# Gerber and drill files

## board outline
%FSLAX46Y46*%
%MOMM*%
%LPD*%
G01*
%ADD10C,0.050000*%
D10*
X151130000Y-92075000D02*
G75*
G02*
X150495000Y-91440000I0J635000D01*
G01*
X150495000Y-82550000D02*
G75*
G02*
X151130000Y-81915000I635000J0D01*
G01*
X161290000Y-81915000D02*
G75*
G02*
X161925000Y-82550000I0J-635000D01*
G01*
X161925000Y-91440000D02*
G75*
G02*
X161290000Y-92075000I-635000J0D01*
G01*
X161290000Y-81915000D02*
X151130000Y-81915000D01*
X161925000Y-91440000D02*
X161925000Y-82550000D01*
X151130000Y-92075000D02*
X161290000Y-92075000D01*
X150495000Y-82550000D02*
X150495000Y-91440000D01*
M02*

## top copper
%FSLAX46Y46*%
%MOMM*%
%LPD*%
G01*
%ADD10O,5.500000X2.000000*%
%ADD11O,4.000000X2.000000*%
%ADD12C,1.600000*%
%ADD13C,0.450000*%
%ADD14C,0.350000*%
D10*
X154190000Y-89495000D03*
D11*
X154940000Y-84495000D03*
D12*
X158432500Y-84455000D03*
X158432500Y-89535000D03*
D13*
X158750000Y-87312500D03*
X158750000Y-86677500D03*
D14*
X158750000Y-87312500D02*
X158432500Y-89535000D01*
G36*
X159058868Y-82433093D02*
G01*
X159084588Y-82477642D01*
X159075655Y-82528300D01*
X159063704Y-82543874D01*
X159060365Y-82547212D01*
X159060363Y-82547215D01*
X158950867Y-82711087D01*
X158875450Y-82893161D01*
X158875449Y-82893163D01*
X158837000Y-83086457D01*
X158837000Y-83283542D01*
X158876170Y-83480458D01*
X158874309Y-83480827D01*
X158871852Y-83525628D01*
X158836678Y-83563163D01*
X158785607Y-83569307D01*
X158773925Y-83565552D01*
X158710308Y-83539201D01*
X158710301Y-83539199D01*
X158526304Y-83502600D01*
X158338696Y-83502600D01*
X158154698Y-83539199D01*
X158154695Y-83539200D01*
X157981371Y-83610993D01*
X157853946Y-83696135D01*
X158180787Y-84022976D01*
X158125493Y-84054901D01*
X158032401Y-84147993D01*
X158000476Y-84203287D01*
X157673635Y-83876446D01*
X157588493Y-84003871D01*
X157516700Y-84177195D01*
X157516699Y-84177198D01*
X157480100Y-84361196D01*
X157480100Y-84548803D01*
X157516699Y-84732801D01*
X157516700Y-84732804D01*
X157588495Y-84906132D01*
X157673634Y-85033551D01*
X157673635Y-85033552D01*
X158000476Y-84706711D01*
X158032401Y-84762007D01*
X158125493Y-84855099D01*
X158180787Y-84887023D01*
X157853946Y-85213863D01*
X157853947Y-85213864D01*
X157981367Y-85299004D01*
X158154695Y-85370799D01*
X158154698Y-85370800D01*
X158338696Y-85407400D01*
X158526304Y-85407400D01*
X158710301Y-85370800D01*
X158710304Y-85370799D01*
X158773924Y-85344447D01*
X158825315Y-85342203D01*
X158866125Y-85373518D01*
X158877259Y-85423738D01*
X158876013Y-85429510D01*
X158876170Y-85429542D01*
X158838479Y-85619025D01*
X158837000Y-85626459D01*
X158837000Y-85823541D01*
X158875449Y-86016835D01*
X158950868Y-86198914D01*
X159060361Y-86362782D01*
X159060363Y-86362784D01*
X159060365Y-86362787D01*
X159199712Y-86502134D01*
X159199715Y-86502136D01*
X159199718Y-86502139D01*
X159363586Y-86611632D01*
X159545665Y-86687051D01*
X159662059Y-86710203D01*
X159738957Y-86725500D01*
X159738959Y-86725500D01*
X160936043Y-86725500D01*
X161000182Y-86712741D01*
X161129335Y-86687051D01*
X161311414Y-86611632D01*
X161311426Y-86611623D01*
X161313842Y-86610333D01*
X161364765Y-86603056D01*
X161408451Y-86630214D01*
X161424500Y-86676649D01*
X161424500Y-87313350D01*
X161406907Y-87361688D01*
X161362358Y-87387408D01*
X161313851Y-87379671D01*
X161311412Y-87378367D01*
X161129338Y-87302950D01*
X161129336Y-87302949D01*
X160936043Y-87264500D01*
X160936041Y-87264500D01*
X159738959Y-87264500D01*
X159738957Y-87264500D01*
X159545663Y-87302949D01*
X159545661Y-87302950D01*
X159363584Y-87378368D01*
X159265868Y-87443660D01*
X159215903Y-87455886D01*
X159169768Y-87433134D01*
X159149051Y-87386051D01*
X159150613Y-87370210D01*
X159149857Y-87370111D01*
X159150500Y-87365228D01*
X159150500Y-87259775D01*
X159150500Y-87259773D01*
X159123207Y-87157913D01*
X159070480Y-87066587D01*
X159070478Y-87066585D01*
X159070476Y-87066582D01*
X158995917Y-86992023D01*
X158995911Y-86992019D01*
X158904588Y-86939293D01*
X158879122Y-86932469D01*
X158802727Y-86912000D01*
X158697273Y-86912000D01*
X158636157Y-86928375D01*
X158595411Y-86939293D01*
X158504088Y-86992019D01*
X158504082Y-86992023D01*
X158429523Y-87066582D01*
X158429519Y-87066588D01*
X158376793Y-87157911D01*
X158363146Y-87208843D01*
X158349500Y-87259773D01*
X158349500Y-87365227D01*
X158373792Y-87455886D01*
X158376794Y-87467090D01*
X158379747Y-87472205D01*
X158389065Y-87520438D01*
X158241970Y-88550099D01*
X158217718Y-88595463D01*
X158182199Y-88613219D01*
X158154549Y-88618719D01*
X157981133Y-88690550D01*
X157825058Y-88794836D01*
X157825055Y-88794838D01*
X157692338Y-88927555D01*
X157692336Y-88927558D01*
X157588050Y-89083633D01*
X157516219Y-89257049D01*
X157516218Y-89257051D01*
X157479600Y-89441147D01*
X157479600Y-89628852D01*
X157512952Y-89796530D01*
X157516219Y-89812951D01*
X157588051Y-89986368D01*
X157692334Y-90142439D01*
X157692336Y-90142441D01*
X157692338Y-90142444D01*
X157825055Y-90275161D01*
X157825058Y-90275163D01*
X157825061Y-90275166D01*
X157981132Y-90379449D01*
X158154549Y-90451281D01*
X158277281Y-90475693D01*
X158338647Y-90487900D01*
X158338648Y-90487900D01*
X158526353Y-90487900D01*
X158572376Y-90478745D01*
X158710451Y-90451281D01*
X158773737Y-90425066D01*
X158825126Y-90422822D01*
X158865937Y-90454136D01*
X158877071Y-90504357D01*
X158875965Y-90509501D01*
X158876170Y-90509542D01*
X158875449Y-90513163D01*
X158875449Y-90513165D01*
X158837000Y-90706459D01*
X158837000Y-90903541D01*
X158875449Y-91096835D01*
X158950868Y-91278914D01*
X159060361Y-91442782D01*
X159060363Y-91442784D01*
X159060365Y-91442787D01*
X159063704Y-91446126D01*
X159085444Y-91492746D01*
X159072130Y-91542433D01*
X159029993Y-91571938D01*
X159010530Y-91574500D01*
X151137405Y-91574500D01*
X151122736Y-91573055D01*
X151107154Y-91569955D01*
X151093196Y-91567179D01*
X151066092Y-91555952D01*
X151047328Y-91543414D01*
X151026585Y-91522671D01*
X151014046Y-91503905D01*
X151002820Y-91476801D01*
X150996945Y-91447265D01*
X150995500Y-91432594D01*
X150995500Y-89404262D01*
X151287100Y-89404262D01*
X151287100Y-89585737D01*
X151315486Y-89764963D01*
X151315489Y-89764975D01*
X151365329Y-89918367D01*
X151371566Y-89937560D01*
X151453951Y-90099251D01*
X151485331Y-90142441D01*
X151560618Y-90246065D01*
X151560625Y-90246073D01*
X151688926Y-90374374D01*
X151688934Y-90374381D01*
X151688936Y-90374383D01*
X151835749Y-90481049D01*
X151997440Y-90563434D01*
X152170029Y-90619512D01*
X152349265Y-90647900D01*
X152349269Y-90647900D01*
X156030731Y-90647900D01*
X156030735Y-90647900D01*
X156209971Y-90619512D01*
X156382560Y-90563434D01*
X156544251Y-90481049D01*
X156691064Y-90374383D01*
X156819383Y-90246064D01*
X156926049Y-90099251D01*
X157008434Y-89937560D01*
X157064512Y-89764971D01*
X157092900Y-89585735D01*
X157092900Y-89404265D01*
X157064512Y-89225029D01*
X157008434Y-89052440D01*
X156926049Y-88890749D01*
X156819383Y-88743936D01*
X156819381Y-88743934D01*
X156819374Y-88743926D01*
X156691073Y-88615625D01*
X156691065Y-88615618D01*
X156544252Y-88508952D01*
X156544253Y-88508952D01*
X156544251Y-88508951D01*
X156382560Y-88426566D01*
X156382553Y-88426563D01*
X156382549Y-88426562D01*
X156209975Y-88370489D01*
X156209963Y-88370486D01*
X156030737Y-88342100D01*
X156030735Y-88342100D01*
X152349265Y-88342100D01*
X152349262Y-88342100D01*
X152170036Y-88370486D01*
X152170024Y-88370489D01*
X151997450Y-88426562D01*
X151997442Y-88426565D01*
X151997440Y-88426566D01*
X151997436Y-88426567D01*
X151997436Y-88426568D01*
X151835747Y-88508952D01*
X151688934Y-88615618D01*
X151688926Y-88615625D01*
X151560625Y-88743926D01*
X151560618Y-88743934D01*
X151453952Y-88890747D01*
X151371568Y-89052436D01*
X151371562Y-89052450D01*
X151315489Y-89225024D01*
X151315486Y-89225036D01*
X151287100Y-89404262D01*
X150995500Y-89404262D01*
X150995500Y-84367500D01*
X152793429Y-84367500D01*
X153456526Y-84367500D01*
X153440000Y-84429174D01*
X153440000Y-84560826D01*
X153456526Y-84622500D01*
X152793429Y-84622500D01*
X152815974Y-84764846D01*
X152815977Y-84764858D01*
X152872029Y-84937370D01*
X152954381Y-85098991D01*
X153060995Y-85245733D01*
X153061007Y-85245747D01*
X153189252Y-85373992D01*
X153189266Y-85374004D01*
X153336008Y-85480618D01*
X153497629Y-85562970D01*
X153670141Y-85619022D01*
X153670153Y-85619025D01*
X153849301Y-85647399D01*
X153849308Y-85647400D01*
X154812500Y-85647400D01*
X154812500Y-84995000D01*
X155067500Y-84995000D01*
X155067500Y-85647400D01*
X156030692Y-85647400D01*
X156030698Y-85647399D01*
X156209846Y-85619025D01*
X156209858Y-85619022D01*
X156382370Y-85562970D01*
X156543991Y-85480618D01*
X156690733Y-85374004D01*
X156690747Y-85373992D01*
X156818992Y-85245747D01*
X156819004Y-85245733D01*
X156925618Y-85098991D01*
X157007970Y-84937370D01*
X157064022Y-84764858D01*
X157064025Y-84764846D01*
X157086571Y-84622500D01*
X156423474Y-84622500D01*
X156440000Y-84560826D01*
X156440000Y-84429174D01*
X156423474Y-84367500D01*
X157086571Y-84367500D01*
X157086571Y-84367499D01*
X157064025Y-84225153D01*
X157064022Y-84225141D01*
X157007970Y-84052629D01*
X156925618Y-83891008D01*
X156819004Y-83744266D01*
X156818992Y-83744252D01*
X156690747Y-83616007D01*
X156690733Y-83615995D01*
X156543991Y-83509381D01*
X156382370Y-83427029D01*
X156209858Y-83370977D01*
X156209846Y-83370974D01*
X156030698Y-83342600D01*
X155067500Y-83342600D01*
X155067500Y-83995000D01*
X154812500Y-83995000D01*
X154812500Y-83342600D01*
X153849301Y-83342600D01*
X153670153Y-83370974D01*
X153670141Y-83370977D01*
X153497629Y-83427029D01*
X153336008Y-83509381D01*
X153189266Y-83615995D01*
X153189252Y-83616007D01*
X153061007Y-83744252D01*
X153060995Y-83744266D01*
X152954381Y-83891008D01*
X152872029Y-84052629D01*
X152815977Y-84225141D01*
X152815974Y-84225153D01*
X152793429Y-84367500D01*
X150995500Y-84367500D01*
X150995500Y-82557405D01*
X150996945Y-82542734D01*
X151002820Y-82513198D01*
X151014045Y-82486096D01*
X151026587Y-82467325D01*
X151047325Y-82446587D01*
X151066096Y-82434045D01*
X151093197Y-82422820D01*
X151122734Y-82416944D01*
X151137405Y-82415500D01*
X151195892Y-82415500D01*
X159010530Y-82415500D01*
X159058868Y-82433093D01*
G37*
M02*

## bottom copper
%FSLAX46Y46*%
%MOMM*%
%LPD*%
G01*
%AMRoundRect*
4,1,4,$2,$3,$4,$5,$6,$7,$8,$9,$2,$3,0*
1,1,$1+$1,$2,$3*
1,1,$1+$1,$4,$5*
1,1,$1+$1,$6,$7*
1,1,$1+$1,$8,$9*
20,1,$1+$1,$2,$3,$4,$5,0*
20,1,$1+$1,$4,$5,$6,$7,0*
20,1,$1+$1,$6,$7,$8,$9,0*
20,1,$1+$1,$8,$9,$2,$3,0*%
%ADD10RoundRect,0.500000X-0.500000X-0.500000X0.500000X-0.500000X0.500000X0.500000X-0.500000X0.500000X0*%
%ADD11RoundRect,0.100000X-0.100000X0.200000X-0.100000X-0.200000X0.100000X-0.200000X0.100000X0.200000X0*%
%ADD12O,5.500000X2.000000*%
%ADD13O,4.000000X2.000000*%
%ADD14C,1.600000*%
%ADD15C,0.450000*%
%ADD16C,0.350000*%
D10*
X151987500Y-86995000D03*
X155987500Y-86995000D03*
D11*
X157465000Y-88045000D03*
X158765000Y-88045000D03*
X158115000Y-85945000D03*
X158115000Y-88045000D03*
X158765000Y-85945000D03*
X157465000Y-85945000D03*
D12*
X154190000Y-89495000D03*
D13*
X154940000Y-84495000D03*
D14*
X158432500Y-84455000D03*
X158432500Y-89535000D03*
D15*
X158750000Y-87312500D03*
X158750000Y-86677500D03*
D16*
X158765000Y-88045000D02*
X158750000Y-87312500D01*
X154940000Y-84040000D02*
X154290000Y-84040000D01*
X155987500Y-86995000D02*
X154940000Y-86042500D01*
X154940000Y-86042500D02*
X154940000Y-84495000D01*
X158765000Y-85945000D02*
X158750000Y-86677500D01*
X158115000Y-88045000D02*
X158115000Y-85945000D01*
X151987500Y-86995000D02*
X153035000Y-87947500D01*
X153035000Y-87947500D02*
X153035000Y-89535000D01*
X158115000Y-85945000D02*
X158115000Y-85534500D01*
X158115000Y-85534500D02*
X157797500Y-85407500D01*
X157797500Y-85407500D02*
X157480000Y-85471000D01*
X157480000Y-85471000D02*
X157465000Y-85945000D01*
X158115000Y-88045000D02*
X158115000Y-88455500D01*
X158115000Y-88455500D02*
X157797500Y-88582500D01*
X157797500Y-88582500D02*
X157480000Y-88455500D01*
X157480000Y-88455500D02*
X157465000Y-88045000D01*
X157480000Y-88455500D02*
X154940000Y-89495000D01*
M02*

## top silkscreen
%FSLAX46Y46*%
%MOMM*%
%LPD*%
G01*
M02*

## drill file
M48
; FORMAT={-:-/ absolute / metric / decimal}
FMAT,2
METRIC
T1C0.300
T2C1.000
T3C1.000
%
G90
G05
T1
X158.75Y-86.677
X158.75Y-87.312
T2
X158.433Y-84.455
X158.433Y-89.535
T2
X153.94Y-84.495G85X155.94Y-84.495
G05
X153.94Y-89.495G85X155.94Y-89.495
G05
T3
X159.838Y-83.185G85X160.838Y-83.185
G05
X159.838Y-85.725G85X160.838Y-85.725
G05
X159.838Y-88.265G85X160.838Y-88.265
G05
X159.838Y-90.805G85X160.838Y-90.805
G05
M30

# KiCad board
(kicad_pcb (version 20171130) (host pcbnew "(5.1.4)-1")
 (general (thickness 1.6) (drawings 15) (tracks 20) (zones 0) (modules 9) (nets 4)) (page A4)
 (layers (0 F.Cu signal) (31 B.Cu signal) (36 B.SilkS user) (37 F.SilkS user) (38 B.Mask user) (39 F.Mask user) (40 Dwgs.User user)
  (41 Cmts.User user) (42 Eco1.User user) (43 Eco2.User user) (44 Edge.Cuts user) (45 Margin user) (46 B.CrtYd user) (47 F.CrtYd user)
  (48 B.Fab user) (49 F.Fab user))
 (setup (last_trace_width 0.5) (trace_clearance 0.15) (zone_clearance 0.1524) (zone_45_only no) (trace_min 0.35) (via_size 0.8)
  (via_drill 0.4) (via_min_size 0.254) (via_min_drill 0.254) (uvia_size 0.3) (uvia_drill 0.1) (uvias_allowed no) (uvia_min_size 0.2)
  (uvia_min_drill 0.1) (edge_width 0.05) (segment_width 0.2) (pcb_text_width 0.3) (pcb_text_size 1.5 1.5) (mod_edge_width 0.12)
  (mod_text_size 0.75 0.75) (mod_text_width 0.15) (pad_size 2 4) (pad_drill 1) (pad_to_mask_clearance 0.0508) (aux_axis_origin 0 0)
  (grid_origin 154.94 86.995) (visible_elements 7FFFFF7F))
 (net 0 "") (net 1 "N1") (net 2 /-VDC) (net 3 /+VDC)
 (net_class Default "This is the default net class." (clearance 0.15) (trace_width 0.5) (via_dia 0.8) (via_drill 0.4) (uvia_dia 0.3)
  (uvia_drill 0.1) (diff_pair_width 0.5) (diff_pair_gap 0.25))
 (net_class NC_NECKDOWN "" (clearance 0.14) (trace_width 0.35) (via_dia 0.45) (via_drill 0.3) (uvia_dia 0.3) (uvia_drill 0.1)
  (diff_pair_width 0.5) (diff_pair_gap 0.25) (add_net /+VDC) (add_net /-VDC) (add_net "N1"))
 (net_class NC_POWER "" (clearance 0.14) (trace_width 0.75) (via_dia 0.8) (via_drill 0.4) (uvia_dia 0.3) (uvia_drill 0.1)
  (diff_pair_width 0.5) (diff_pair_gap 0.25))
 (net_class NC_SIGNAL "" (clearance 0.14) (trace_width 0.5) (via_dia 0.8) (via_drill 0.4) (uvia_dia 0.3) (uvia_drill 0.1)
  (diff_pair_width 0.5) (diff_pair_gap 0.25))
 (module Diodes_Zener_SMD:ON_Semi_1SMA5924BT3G (layer B.Cu) (at 153.9875 86.995)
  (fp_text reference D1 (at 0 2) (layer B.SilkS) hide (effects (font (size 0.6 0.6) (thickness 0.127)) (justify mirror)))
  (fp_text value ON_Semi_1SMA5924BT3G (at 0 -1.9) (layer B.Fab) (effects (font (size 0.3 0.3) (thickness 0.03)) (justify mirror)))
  (pad 2 smd roundrect (at -2 0) (size 2 2) (layers B.Cu B.Paste B.Mask) (roundrect_rratio 0.25) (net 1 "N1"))
  (pad 1 smd roundrect (at 2 0) (size 2 2) (layers B.Cu B.Paste B.Mask) (roundrect_rratio 0.25) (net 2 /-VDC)))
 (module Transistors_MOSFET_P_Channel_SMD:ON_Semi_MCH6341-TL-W (layer B.Cu) (at 158.115 86.995 270)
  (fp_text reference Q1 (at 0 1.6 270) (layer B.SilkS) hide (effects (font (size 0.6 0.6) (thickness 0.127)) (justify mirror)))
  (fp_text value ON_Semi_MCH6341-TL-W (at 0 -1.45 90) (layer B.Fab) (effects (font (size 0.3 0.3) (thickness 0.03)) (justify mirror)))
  (pad 6 smd roundrect (at 1.05 0.65 270) (size 0.6 0.4) (layers B.Cu B.Paste B.Mask) (roundrect_rratio 0.25) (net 1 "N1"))
  (pad 4 smd roundrect (at 1.05 -0.65 270) (size 0.6 0.4) (layers B.Cu B.Paste B.Mask) (roundrect_rratio 0.25) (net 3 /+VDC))
  (pad 2 smd roundrect (at -1.05 0 270) (size 0.6 0.4) (layers B.Cu B.Paste B.Mask) (roundrect_rratio 0.25) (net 1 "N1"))
  (pad 5 smd roundrect (at 1.05 0 270) (size 0.6 0.4) (layers B.Cu B.Paste B.Mask) (roundrect_rratio 0.25) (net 1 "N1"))
  (pad 3 smd roundrect (at -1.05 -0.65 270) (size 0.6 0.4) (layers B.Cu B.Paste B.Mask) (roundrect_rratio 0.25) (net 2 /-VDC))
  (pad 1 smd roundrect (at -1.05 0.65 270) (size 0.6 0.4) (layers B.Cu B.Paste B.Mask) (roundrect_rratio 0.25) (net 1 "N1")))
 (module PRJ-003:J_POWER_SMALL (layer F.Cu) (at 154.94 86.995)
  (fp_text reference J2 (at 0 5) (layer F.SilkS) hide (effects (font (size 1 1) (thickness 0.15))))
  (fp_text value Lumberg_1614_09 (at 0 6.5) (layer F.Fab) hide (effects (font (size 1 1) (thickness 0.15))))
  (pad 2 thru_hole oval (at 0 2.5) (size 5.5 2) (drill oval 3 1 (offset -0.75 0)) (layers *.Cu *.Mask) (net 1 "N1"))
  (pad 1 thru_hole oval (at 0 -2.5 90) (size 2 4) (drill oval 1 3) (layers *.Cu *.Mask) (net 2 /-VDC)))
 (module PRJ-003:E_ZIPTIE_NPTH (layer F.Cu) (at 160.3375 88.265 90)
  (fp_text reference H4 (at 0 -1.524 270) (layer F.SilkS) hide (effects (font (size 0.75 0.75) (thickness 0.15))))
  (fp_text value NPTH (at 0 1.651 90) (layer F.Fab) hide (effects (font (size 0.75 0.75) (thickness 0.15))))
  (pad "" np_thru_hole oval (at 0 0 90) (size 1 2) (drill oval 1 2) (layers *.Cu *.Mask)))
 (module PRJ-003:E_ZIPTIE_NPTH (layer F.Cu) (at 160.3375 85.725 90)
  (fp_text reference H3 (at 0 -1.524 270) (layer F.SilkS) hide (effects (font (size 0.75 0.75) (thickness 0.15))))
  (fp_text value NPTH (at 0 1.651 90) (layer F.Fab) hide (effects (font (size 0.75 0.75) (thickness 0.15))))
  (pad "" np_thru_hole oval (at 0 0 90) (size 1 2) (drill oval 1 2) (layers *.Cu *.Mask)))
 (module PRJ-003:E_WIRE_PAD (layer B.Cu) (at 158.4325 84.455)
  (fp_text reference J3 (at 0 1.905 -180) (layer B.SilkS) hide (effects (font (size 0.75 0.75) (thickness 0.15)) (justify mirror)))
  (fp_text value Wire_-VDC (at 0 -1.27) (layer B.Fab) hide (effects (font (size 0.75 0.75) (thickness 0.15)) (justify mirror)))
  (pad "" connect circle (at 0 0) (size 1 1) (layers B.Mask))
  (pad 1 thru_hole circle (at 0 0) (size 1.6 1.6) (drill 1) (layers F.Cu F.Mask) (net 2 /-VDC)))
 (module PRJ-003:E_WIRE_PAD (layer B.Cu) (at 158.4325 89.535)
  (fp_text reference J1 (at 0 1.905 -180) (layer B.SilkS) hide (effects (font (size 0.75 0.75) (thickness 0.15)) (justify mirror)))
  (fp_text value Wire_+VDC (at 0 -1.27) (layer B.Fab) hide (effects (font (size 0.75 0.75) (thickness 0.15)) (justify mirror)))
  (pad "" connect circle (at 0 0) (size 1 1) (layers B.Mask))
  (pad 1 thru_hole circle (at 0 0) (size 1.6 1.6) (drill 1) (layers F.Cu F.Mask) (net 3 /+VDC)))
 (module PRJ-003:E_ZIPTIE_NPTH (layer F.Cu) (at 160.3375 90.805 90)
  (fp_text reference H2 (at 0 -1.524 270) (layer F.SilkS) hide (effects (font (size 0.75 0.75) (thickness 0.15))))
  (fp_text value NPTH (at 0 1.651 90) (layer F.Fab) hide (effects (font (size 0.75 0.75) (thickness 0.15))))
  (pad "" np_thru_hole oval (at 0 0 90) (size 1 2) (drill oval 1 2) (layers *.Cu *.Mask)))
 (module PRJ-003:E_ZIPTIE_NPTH (layer F.Cu) (at 160.3375 83.185 90)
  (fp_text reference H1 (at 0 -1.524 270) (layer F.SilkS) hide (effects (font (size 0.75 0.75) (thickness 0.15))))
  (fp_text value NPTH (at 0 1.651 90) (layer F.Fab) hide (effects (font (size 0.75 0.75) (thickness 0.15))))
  (pad "" np_thru_hole oval (at 0 0 90) (size 1 2) (drill oval 1 2) (layers *.Cu *.Mask)))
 (gr_arc (start 151.13 91.44) (end 150.495 91.44) (angle -90) (layer Edge.Cuts) (width 0.05))
 (gr_arc (start 151.13 82.55) (end 151.13 81.915) (angle -90) (layer Edge.Cuts) (width 0.05))
 (gr_arc (start 161.29 82.55) (end 161.925 82.55) (angle -90) (layer Edge.Cuts) (width 0.05))
 (gr_arc (start 161.29 91.44) (end 161.29 92.075) (angle -90) (layer Edge.Cuts) (width 0.05))
 (gr_line (start 161.29 81.915) (end 151.13 81.915) (layer Edge.Cuts) (width 0.05))
 (gr_line (start 161.925 91.44) (end 161.925 82.55) (layer Edge.Cuts) (width 0.05))
 (gr_line (start 151.13 92.075) (end 161.29 92.075) (layer Edge.Cuts) (width 0.05))
 (gr_line (start 150.495 82.55) (end 150.495 91.44) (layer Edge.Cuts) (width 0.05))
 (via (at 158.75 87.3125) (size 0.45) (drill 0.3) (layers F.Cu B.Cu) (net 3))
 (segment (start 158.765 88.045) (end 158.75 87.3125) (width 0.35) (layer B.Cu) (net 3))
 (segment (start 158.75 87.3125) (end 158.4325 89.535) (width 0.35) (layer F.Cu) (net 3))
 (segment (start 154.94 84.04) (end 154.29 84.04) (width 0.35) (layer B.Cu) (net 2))
 (segment (start 155.9875 86.995) (end 154.94 86.0425) (width 0.35) (layer B.Cu) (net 2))
 (segment (start 154.94 86.0425) (end 154.94 84.495) (width 0.35) (layer B.Cu) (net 2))
 (segment (start 158.765 85.945) (end 158.75 86.6775) (width 0.35) (layer B.Cu) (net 2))
 (via (at 158.75 86.6775) (size 0.45) (drill 0.3) (layers F.Cu B.Cu) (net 2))
 (segment (start 158.115 88.045) (end 158.115 85.945) (width 0.35) (layer B.Cu) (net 1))
 (segment (start 151.9875 86.995) (end 153.035 87.9475) (width 0.35) (layer B.Cu) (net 1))
 (segment (start 153.035 87.9475) (end 153.035 89.535) (width 0.35) (layer B.Cu) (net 1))
 (segment (start 158.115 85.945) (end 158.115 85.5345) (width 0.35) (layer B.Cu) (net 1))
 (segment (start 158.115 85.5345) (end 157.7975 85.4075) (width 0.35) (layer B.Cu) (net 1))
 (segment (start 157.7975 85.4075) (end 157.48 85.471) (width 0.35) (layer B.Cu) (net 1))
 (segment (start 157.48 85.471) (end 157.465 85.945) (width 0.35) (layer B.Cu) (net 1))
 (segment (start 158.115 88.045) (end 158.115 88.4555) (width 0.35) (layer B.Cu) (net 1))
 (segment (start 158.115 88.4555) (end 157.7975 88.5825) (width 0.35) (layer B.Cu) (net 1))
 (segment (start 157.7975 88.5825) (end 157.48 88.4555) (width 0.35) (layer B.Cu) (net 1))
 (segment (start 157.48 88.4555) (end 157.465 88.045) (width 0.35) (layer B.Cu) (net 1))
 (segment (start 157.48 88.4555) (end 154.94 89.495) (width 0.35) (layer B.Cu) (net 1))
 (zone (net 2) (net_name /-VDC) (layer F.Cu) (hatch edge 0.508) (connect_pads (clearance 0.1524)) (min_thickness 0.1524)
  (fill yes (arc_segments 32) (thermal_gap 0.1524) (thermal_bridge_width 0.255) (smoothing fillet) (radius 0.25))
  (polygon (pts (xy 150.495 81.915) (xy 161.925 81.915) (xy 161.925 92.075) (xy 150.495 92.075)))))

